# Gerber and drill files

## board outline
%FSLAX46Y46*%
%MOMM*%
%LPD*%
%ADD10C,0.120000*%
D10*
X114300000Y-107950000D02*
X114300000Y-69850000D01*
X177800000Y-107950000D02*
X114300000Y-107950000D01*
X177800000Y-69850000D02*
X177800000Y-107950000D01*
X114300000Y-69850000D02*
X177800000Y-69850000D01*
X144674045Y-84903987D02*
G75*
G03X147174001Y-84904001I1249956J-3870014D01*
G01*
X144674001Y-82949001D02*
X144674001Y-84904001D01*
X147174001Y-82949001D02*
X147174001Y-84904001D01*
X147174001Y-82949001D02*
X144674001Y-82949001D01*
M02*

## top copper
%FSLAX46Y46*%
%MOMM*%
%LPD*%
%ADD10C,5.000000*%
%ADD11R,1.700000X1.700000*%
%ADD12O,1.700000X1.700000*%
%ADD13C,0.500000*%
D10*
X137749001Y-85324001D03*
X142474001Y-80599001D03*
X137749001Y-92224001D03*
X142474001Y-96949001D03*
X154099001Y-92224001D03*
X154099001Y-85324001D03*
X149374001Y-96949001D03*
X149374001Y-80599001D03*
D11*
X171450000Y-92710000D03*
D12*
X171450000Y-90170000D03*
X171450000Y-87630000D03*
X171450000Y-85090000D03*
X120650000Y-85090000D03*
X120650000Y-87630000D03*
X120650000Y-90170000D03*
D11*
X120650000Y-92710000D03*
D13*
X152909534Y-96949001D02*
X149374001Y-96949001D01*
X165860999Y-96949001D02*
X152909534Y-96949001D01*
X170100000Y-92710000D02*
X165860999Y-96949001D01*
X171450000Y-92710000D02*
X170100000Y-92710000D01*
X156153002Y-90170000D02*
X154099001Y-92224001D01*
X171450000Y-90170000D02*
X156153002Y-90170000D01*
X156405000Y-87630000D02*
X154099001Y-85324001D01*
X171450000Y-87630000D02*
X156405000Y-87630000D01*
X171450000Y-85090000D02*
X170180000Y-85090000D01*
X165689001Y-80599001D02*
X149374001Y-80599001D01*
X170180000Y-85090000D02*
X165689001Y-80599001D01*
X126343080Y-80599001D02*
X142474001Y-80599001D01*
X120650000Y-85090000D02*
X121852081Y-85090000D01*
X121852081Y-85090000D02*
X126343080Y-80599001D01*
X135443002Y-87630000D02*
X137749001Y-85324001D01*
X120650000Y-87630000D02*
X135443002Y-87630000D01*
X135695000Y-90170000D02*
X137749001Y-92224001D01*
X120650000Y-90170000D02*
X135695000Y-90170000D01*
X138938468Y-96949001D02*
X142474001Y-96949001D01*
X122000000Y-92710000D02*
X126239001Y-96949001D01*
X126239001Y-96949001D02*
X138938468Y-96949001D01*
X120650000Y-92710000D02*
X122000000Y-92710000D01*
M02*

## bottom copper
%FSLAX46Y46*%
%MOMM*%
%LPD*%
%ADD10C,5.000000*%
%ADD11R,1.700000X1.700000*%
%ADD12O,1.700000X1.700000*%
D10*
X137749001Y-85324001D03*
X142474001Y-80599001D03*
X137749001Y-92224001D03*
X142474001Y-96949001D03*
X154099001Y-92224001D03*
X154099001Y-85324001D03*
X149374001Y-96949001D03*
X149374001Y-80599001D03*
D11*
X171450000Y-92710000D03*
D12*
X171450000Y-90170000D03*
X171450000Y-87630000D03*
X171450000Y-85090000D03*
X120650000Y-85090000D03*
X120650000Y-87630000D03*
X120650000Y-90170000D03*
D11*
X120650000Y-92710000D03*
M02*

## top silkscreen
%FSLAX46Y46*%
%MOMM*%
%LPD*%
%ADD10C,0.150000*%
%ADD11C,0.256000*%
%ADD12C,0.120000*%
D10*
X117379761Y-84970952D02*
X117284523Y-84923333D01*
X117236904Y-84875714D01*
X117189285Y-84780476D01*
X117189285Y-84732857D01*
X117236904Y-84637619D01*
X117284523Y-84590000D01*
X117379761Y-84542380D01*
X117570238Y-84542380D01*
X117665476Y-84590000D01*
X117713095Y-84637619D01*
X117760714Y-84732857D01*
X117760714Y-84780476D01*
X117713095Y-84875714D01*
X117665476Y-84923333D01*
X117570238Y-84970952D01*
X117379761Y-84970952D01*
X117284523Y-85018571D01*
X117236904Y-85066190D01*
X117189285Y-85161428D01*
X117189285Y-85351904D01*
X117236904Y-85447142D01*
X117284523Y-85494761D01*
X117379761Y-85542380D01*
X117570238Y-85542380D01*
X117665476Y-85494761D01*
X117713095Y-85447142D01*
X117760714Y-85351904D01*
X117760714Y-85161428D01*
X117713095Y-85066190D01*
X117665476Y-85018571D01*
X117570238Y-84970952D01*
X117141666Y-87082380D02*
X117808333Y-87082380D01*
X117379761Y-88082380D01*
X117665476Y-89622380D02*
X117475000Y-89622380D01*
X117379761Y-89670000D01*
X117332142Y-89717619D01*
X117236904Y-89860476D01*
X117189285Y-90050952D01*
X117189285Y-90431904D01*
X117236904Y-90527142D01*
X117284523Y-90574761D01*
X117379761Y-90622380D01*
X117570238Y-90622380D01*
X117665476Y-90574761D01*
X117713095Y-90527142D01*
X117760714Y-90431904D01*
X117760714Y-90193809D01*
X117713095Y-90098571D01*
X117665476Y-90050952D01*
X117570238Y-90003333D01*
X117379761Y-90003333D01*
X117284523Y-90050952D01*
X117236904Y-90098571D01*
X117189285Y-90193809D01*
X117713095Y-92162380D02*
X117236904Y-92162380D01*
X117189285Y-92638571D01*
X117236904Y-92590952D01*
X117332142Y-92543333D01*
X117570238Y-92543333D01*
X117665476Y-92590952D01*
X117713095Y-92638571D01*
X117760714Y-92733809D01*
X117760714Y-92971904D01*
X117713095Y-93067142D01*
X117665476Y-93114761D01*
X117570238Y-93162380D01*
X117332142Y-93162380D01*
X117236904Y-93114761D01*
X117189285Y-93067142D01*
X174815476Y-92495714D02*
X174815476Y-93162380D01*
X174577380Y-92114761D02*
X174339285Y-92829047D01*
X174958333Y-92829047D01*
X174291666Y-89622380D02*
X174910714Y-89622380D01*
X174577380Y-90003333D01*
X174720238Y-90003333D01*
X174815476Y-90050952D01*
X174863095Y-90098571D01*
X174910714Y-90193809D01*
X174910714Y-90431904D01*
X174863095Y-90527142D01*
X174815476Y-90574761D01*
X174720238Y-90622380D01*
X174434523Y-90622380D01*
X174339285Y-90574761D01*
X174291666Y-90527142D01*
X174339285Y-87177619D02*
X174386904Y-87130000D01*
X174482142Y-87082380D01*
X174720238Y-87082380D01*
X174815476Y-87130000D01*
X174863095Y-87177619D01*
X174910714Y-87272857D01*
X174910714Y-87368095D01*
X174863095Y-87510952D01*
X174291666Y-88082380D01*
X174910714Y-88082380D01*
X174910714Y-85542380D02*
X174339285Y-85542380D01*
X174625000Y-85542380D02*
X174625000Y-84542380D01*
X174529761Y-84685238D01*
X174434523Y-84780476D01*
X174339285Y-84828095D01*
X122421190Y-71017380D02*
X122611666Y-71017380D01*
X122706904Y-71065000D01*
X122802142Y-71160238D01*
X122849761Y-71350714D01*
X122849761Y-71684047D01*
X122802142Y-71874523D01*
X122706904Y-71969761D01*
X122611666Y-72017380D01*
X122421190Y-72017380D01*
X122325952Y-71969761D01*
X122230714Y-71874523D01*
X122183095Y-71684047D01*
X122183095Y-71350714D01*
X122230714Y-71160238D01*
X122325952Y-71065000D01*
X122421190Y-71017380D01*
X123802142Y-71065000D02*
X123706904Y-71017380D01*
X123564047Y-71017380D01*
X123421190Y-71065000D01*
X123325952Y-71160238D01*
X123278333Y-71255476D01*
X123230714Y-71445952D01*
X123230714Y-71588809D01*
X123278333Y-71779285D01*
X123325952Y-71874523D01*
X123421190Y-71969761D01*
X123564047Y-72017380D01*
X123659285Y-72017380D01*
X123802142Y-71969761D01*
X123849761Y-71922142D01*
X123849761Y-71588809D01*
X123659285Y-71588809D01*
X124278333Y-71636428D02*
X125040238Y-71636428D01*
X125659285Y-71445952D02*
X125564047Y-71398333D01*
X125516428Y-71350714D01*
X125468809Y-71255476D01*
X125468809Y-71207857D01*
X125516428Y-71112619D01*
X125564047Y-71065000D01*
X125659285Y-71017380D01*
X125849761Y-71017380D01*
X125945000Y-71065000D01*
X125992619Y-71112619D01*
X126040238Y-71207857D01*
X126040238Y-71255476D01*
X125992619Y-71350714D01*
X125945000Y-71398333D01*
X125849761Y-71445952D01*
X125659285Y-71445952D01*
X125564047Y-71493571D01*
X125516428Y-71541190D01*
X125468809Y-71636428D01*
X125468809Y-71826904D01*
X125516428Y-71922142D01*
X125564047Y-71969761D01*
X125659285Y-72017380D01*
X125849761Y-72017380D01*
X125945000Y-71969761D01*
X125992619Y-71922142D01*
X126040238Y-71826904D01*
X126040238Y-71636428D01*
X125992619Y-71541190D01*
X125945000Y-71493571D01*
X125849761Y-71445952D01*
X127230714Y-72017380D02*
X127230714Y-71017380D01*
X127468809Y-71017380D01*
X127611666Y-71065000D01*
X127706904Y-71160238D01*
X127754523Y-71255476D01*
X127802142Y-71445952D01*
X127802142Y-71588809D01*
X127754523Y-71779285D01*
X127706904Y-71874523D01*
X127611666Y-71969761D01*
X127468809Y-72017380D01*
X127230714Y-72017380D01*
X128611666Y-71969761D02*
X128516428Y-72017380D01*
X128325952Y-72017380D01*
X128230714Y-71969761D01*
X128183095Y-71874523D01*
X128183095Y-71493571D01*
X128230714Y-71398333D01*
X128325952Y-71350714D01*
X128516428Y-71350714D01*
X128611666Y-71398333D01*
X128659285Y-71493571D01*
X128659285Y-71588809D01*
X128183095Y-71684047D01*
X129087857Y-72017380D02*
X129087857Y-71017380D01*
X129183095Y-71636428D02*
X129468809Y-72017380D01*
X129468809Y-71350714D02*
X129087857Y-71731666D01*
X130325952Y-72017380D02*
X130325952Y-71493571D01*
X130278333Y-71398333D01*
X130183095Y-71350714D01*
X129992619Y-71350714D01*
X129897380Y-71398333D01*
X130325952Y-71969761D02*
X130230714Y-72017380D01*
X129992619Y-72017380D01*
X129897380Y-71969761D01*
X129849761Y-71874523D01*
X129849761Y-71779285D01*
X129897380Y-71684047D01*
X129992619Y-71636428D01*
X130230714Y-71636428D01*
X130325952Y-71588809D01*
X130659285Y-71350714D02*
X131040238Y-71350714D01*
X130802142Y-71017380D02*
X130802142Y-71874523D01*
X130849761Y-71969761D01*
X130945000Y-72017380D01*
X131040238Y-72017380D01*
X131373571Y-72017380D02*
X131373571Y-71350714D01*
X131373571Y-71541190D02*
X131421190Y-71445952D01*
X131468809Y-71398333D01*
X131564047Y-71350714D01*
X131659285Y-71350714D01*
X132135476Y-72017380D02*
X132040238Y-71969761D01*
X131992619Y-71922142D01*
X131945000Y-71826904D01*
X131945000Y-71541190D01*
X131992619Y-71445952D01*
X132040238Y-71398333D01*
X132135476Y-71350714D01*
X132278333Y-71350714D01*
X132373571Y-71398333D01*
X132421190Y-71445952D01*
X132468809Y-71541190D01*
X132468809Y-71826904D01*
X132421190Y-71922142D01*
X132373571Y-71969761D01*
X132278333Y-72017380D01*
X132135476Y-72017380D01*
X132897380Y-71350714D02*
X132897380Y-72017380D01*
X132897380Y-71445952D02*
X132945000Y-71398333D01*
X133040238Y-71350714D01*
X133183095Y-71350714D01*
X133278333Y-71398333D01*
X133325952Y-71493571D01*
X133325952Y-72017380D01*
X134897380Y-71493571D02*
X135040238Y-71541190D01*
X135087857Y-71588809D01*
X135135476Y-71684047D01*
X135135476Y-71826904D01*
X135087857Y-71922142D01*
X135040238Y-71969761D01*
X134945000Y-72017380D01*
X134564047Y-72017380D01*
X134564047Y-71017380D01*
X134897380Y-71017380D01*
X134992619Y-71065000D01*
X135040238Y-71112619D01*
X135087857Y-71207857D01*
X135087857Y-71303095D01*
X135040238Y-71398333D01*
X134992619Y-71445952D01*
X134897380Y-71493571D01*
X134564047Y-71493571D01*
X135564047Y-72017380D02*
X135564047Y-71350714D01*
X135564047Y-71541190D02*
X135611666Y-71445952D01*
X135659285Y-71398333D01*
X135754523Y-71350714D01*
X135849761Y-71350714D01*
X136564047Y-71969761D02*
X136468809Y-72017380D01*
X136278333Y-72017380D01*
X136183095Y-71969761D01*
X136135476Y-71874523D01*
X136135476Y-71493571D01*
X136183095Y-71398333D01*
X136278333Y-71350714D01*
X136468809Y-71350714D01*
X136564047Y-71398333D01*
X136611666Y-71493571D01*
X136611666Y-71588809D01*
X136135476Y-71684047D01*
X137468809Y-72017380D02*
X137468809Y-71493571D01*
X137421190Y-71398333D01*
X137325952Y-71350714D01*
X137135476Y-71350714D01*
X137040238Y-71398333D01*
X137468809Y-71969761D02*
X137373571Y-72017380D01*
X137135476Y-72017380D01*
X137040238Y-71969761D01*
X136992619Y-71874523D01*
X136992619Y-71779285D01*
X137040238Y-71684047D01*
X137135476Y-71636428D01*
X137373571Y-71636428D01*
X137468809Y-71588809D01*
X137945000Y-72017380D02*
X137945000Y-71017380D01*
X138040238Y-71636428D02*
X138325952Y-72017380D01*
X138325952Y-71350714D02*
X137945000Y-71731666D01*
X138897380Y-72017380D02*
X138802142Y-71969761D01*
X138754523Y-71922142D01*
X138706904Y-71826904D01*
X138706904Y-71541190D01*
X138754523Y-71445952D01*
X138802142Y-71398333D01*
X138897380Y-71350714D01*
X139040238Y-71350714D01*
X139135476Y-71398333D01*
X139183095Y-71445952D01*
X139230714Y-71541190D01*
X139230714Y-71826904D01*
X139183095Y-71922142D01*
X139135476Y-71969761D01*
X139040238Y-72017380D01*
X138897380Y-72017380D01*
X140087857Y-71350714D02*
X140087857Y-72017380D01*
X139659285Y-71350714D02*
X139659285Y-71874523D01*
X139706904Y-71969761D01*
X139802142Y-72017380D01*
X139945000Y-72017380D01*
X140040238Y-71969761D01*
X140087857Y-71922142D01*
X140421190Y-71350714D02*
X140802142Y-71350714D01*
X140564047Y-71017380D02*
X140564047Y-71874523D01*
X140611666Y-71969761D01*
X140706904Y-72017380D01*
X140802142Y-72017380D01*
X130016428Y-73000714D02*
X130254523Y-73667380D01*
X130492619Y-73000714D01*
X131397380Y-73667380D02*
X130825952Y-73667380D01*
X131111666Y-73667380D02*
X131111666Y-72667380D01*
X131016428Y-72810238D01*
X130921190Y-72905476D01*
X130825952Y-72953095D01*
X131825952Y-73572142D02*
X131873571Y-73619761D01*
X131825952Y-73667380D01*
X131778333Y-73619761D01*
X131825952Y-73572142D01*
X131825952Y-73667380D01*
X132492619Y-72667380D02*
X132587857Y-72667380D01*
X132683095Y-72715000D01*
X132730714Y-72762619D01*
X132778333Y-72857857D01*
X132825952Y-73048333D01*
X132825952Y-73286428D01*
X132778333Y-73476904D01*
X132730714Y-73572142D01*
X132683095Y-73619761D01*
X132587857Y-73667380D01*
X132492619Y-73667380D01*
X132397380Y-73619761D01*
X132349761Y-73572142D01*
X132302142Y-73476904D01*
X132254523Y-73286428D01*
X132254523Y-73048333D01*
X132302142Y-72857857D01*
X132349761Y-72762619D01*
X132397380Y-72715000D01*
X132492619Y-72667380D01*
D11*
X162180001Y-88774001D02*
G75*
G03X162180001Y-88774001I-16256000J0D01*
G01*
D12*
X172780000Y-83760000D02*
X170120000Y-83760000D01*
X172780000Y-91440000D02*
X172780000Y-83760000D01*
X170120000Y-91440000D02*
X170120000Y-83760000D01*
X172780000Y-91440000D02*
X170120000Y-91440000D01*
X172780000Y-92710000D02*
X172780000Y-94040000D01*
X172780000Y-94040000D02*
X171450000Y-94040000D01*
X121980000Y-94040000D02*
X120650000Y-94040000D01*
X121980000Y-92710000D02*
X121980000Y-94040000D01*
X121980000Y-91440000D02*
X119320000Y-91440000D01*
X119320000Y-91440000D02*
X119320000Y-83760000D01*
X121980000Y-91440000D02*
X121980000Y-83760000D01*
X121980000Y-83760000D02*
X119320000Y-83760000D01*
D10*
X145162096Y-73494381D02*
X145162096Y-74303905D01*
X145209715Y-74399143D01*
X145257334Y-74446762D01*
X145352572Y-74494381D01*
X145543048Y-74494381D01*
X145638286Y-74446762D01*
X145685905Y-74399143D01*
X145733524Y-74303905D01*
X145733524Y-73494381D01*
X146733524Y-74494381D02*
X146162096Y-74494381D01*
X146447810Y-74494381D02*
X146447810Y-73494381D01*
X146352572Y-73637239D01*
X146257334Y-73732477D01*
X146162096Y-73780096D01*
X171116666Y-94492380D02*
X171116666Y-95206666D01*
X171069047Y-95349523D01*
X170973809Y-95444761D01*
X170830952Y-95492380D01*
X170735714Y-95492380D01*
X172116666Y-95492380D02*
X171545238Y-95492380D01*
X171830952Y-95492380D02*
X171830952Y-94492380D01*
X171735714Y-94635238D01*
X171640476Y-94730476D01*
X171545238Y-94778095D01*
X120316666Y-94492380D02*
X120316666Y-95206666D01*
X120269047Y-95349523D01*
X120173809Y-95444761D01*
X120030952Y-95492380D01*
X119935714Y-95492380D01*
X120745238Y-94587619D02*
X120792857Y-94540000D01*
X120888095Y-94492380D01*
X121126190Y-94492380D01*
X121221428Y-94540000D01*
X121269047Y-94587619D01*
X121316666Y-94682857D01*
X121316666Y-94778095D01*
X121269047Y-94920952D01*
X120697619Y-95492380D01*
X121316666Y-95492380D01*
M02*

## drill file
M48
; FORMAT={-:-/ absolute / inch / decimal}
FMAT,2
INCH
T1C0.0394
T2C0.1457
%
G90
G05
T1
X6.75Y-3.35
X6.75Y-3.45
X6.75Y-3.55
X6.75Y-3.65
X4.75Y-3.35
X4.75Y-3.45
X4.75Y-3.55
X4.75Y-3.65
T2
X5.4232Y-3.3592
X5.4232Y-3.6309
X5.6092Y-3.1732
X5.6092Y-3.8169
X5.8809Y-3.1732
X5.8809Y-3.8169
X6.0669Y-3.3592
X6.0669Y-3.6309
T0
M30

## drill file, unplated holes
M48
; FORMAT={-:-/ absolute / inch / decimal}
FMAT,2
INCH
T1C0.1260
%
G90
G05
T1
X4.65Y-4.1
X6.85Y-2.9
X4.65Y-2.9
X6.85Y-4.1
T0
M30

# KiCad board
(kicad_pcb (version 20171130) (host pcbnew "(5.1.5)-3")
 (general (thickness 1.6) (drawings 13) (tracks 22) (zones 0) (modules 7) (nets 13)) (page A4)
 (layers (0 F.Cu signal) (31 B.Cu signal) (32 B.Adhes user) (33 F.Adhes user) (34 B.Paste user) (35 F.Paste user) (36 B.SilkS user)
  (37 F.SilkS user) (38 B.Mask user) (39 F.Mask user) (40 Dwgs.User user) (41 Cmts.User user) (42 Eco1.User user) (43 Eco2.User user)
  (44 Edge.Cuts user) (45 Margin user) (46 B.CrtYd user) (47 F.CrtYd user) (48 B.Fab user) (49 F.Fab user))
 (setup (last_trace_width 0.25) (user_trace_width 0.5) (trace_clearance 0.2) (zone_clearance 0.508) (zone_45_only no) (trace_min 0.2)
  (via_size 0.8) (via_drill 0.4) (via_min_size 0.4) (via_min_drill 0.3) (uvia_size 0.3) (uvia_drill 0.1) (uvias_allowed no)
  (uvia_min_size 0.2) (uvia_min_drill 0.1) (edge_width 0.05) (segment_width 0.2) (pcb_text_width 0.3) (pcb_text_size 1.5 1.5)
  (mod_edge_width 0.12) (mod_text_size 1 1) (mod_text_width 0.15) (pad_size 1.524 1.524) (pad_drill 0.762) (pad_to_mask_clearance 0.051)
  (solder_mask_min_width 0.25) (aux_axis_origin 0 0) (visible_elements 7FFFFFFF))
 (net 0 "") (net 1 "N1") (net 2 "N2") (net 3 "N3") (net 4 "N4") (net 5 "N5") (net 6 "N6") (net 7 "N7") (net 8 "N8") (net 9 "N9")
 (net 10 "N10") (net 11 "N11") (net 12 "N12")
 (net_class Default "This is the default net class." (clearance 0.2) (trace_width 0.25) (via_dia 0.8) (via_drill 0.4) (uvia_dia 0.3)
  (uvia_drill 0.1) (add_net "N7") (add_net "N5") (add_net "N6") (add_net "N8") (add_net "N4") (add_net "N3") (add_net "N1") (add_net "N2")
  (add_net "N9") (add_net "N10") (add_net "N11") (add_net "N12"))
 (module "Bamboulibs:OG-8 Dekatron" (layer F.Cu) (at 145.924001 88.774001)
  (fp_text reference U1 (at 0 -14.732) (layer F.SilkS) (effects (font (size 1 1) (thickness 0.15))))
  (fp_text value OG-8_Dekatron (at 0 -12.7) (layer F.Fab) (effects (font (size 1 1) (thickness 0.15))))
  (fp_arc (start 0 0) (end 1.25 -3.87) (angle 324.2) (layer Edge.Cuts) (width 0.12))
  (fp_line (start -1.25 -5.825) (end -1.25 -3.87) (layer Edge.Cuts) (width 0.12))
  (fp_line (start 1.25 -5.825) (end 1.25 -3.87) (layer Edge.Cuts) (width 0.12))
  (fp_line (start 1.25 -5.825) (end -1.25 -5.825) (layer Edge.Cuts) (width 0.12))
  (fp_circle (center 0 0) (end 16.256 0) (layer F.SilkS) (width 0.256))
  (pad 7 thru_hole circle (at -8.175 -3.45) (size 5 5) (drill 3.7) (layers *.Cu *.Mask) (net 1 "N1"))
  (pad 8 thru_hole circle (at -3.45 -8.175) (size 5 5) (drill 3.7) (layers *.Cu *.Mask) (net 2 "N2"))
  (pad 6 thru_hole circle (at -8.175 3.45) (size 5 5) (drill 3.7) (layers *.Cu *.Mask) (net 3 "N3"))
  (pad 5 thru_hole circle (at -3.45 8.175) (size 5 5) (drill 3.7) (layers *.Cu *.Mask) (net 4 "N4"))
  (pad 3 thru_hole circle (at 8.175 3.45) (size 5 5) (drill 3.7) (layers *.Cu *.Mask) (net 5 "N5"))
  (pad 2 thru_hole circle (at 8.175 -3.45) (size 5 5) (drill 3.7) (layers *.Cu *.Mask) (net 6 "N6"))
  (pad 4 thru_hole circle (at 3.45 8.175) (size 5 5) (drill 3.7) (layers *.Cu *.Mask) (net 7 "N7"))
  (pad 1 thru_hole circle (at 3.45 -8.175) (size 5 5) (drill 3.7) (layers *.Cu *.Mask) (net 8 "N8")))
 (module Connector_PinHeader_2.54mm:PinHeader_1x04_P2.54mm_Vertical (layer F.Cu) (at 171.45 92.71 180)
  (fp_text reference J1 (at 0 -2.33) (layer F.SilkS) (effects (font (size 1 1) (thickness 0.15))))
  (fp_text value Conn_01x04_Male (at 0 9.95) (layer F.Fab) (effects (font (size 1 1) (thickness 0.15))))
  (fp_line (start -1.33 8.95) (end 1.33 8.95) (layer F.SilkS) (width 0.12))
  (fp_line (start -1.33 1.27) (end -1.33 8.95) (layer F.SilkS) (width 0.12))
  (fp_line (start 1.33 1.27) (end 1.33 8.95) (layer F.SilkS) (width 0.12))
  (fp_line (start -1.33 1.27) (end 1.33 1.27) (layer F.SilkS) (width 0.12))
  (fp_line (start -1.33 0) (end -1.33 -1.33) (layer F.SilkS) (width 0.12))
  (fp_line (start -1.33 -1.33) (end 0 -1.33) (layer F.SilkS) (width 0.12))
  (pad 1 thru_hole rect (at 0 0 180) (size 1.7 1.7) (drill 1) (layers *.Cu *.Mask) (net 7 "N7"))
  (pad 2 thru_hole oval (at 0 2.54 180) (size 1.7 1.7) (drill 1) (layers *.Cu *.Mask) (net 5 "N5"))
  (pad 3 thru_hole oval (at 0 5.08 180) (size 1.7 1.7) (drill 1) (layers *.Cu *.Mask) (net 6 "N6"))
  (pad 4 thru_hole oval (at 0 7.62 180) (size 1.7 1.7) (drill 1) (layers *.Cu *.Mask) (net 8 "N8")))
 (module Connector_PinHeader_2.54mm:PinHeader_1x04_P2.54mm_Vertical (layer F.Cu) (at 120.65 92.71 180)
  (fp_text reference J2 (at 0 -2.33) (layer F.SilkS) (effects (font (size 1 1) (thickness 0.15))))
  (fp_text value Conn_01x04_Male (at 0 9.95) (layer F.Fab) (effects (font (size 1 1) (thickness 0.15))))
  (fp_line (start -1.33 -1.33) (end 0 -1.33) (layer F.SilkS) (width 0.12))
  (fp_line (start -1.33 0) (end -1.33 -1.33) (layer F.SilkS) (width 0.12))
  (fp_line (start -1.33 1.27) (end 1.33 1.27) (layer F.SilkS) (width 0.12))
  (fp_line (start 1.33 1.27) (end 1.33 8.95) (layer F.SilkS) (width 0.12))
  (fp_line (start -1.33 1.27) (end -1.33 8.95) (layer F.SilkS) (width 0.12))
  (fp_line (start -1.33 8.95) (end 1.33 8.95) (layer F.SilkS) (width 0.12))
  (pad 4 thru_hole oval (at 0 7.62 180) (size 1.7 1.7) (drill 1) (layers *.Cu *.Mask) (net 2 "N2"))
  (pad 3 thru_hole oval (at 0 5.08 180) (size 1.7 1.7) (drill 1) (layers *.Cu *.Mask) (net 1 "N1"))
  (pad 2 thru_hole oval (at 0 2.54 180) (size 1.7 1.7) (drill 1) (layers *.Cu *.Mask) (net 3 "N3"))
  (pad 1 thru_hole rect (at 0 0 180) (size 1.7 1.7) (drill 1) (layers *.Cu *.Mask) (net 4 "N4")))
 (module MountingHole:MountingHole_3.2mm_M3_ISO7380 (layer F.Cu) (at 118.11 73.66)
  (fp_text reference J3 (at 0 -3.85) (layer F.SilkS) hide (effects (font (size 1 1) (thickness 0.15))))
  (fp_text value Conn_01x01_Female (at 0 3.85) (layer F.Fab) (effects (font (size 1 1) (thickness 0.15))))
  (pad 1 np_thru_hole circle (at 0 0) (size 3.2 3.2) (drill 3.2) (layers *.Cu *.Mask) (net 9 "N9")))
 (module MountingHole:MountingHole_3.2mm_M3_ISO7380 (layer F.Cu) (at 173.99 73.66)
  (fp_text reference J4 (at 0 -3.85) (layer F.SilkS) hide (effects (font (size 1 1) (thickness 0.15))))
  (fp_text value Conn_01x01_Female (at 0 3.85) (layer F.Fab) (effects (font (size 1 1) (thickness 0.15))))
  (pad 1 np_thru_hole circle (at 0 0) (size 3.2 3.2) (drill 3.2) (layers *.Cu *.Mask) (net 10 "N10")))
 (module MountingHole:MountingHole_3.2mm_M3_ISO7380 (layer F.Cu) (at 118.11 104.14)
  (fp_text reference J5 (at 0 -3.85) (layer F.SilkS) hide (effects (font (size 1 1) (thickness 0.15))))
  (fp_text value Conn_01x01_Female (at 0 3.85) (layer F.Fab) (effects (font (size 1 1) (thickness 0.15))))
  (pad 1 np_thru_hole circle (at 0 0) (size 3.2 3.2) (drill 3.2) (layers *.Cu *.Mask) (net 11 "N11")))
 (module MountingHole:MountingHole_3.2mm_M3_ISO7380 (layer F.Cu) (at 173.99 104.14)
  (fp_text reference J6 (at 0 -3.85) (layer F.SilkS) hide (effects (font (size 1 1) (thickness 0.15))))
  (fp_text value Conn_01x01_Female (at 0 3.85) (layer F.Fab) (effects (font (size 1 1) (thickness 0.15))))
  (pad 1 np_thru_hole circle (at 0 0) (size 3.2 3.2) (drill 3.2) (layers *.Cu *.Mask) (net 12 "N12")))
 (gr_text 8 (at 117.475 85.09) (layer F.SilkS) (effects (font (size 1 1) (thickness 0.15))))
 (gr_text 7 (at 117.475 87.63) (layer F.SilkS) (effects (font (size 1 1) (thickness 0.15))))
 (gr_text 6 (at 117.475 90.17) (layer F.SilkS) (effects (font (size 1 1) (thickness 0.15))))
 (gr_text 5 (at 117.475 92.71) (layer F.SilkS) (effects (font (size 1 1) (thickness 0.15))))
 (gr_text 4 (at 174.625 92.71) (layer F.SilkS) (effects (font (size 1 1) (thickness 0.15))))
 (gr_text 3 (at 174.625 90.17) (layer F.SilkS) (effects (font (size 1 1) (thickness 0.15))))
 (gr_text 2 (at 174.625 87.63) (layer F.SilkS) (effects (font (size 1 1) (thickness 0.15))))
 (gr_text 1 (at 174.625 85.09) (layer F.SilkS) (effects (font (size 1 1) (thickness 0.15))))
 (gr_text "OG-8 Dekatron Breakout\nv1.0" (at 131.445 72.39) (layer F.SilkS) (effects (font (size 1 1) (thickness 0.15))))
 (gr_line (start 114.3 107.95) (end 114.3 69.85) (layer Edge.Cuts) (width 0.12))
 (gr_line (start 177.8 107.95) (end 114.3 107.95) (layer Edge.Cuts) (width 0.12))
 (gr_line (start 177.8 69.85) (end 177.8 107.95) (layer Edge.Cuts) (width 0.12))
 (gr_line (start 114.3 69.85) (end 177.8 69.85) (layer Edge.Cuts) (width 0.12))
 (segment (start 152.909534 96.949001) (end 149.374001 96.949001) (width 0.5) (layer F.Cu) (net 7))
 (segment (start 165.860999 96.949001) (end 152.909534 96.949001) (width 0.5) (layer F.Cu) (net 7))
 (segment (start 170.1 92.71) (end 165.860999 96.949001) (width 0.5) (layer F.Cu) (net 7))
 (segment (start 171.45 92.71) (end 170.1 92.71) (width 0.5) (layer F.Cu) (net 7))
 (segment (start 156.153002 90.17) (end 154.099001 92.224001) (width 0.5) (layer F.Cu) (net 5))
 (segment (start 171.45 90.17) (end 156.153002 90.17) (width 0.5) (layer F.Cu) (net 5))
 (segment (start 156.405 87.63) (end 154.099001 85.324001) (width 0.5) (layer F.Cu) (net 6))
 (segment (start 171.45 87.63) (end 156.405 87.63) (width 0.5) (layer F.Cu) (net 6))
 (segment (start 171.45 85.09) (end 170.18 85.09) (width 0.5) (layer F.Cu) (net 8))
 (segment (start 165.689001 80.599001) (end 149.374001 80.599001) (width 0.5) (layer F.Cu) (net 8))
 (segment (start 170.18 85.09) (end 165.689001 80.599001) (width 0.5) (layer F.Cu) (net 8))
 (segment (start 126.34308 80.599001) (end 142.474001 80.599001) (width 0.5) (layer F.Cu) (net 2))
 (segment (start 120.65 85.09) (end 121.852081 85.09) (width 0.5) (layer F.Cu) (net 2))
 (segment (start 121.852081 85.09) (end 126.34308 80.599001) (width 0.5) (layer F.Cu) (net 2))
 (segment (start 135.443002 87.63) (end 137.749001 85.324001) (width 0.5) (layer F.Cu) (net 1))
 (segment (start 120.65 87.63) (end 135.443002 87.63) (width 0.5) (layer F.Cu) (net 1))
 (segment (start 135.695 90.17) (end 137.749001 92.224001) (width 0.5) (layer F.Cu) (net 3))
 (segment (start 120.65 90.17) (end 135.695 90.17) (width 0.5) (layer F.Cu) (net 3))
 (segment (start 138.938468 96.949001) (end 142.474001 96.949001) (width 0.5) (layer F.Cu) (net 4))
 (segment (start 122 92.71) (end 126.239001 96.949001) (width 0.5) (layer F.Cu) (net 4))
 (segment (start 126.239001 96.949001) (end 138.938468 96.949001) (width 0.5) (layer F.Cu) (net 4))
 (segment (start 120.65 92.71) (end 122 92.71) (width 0.5) (layer F.Cu) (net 4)))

